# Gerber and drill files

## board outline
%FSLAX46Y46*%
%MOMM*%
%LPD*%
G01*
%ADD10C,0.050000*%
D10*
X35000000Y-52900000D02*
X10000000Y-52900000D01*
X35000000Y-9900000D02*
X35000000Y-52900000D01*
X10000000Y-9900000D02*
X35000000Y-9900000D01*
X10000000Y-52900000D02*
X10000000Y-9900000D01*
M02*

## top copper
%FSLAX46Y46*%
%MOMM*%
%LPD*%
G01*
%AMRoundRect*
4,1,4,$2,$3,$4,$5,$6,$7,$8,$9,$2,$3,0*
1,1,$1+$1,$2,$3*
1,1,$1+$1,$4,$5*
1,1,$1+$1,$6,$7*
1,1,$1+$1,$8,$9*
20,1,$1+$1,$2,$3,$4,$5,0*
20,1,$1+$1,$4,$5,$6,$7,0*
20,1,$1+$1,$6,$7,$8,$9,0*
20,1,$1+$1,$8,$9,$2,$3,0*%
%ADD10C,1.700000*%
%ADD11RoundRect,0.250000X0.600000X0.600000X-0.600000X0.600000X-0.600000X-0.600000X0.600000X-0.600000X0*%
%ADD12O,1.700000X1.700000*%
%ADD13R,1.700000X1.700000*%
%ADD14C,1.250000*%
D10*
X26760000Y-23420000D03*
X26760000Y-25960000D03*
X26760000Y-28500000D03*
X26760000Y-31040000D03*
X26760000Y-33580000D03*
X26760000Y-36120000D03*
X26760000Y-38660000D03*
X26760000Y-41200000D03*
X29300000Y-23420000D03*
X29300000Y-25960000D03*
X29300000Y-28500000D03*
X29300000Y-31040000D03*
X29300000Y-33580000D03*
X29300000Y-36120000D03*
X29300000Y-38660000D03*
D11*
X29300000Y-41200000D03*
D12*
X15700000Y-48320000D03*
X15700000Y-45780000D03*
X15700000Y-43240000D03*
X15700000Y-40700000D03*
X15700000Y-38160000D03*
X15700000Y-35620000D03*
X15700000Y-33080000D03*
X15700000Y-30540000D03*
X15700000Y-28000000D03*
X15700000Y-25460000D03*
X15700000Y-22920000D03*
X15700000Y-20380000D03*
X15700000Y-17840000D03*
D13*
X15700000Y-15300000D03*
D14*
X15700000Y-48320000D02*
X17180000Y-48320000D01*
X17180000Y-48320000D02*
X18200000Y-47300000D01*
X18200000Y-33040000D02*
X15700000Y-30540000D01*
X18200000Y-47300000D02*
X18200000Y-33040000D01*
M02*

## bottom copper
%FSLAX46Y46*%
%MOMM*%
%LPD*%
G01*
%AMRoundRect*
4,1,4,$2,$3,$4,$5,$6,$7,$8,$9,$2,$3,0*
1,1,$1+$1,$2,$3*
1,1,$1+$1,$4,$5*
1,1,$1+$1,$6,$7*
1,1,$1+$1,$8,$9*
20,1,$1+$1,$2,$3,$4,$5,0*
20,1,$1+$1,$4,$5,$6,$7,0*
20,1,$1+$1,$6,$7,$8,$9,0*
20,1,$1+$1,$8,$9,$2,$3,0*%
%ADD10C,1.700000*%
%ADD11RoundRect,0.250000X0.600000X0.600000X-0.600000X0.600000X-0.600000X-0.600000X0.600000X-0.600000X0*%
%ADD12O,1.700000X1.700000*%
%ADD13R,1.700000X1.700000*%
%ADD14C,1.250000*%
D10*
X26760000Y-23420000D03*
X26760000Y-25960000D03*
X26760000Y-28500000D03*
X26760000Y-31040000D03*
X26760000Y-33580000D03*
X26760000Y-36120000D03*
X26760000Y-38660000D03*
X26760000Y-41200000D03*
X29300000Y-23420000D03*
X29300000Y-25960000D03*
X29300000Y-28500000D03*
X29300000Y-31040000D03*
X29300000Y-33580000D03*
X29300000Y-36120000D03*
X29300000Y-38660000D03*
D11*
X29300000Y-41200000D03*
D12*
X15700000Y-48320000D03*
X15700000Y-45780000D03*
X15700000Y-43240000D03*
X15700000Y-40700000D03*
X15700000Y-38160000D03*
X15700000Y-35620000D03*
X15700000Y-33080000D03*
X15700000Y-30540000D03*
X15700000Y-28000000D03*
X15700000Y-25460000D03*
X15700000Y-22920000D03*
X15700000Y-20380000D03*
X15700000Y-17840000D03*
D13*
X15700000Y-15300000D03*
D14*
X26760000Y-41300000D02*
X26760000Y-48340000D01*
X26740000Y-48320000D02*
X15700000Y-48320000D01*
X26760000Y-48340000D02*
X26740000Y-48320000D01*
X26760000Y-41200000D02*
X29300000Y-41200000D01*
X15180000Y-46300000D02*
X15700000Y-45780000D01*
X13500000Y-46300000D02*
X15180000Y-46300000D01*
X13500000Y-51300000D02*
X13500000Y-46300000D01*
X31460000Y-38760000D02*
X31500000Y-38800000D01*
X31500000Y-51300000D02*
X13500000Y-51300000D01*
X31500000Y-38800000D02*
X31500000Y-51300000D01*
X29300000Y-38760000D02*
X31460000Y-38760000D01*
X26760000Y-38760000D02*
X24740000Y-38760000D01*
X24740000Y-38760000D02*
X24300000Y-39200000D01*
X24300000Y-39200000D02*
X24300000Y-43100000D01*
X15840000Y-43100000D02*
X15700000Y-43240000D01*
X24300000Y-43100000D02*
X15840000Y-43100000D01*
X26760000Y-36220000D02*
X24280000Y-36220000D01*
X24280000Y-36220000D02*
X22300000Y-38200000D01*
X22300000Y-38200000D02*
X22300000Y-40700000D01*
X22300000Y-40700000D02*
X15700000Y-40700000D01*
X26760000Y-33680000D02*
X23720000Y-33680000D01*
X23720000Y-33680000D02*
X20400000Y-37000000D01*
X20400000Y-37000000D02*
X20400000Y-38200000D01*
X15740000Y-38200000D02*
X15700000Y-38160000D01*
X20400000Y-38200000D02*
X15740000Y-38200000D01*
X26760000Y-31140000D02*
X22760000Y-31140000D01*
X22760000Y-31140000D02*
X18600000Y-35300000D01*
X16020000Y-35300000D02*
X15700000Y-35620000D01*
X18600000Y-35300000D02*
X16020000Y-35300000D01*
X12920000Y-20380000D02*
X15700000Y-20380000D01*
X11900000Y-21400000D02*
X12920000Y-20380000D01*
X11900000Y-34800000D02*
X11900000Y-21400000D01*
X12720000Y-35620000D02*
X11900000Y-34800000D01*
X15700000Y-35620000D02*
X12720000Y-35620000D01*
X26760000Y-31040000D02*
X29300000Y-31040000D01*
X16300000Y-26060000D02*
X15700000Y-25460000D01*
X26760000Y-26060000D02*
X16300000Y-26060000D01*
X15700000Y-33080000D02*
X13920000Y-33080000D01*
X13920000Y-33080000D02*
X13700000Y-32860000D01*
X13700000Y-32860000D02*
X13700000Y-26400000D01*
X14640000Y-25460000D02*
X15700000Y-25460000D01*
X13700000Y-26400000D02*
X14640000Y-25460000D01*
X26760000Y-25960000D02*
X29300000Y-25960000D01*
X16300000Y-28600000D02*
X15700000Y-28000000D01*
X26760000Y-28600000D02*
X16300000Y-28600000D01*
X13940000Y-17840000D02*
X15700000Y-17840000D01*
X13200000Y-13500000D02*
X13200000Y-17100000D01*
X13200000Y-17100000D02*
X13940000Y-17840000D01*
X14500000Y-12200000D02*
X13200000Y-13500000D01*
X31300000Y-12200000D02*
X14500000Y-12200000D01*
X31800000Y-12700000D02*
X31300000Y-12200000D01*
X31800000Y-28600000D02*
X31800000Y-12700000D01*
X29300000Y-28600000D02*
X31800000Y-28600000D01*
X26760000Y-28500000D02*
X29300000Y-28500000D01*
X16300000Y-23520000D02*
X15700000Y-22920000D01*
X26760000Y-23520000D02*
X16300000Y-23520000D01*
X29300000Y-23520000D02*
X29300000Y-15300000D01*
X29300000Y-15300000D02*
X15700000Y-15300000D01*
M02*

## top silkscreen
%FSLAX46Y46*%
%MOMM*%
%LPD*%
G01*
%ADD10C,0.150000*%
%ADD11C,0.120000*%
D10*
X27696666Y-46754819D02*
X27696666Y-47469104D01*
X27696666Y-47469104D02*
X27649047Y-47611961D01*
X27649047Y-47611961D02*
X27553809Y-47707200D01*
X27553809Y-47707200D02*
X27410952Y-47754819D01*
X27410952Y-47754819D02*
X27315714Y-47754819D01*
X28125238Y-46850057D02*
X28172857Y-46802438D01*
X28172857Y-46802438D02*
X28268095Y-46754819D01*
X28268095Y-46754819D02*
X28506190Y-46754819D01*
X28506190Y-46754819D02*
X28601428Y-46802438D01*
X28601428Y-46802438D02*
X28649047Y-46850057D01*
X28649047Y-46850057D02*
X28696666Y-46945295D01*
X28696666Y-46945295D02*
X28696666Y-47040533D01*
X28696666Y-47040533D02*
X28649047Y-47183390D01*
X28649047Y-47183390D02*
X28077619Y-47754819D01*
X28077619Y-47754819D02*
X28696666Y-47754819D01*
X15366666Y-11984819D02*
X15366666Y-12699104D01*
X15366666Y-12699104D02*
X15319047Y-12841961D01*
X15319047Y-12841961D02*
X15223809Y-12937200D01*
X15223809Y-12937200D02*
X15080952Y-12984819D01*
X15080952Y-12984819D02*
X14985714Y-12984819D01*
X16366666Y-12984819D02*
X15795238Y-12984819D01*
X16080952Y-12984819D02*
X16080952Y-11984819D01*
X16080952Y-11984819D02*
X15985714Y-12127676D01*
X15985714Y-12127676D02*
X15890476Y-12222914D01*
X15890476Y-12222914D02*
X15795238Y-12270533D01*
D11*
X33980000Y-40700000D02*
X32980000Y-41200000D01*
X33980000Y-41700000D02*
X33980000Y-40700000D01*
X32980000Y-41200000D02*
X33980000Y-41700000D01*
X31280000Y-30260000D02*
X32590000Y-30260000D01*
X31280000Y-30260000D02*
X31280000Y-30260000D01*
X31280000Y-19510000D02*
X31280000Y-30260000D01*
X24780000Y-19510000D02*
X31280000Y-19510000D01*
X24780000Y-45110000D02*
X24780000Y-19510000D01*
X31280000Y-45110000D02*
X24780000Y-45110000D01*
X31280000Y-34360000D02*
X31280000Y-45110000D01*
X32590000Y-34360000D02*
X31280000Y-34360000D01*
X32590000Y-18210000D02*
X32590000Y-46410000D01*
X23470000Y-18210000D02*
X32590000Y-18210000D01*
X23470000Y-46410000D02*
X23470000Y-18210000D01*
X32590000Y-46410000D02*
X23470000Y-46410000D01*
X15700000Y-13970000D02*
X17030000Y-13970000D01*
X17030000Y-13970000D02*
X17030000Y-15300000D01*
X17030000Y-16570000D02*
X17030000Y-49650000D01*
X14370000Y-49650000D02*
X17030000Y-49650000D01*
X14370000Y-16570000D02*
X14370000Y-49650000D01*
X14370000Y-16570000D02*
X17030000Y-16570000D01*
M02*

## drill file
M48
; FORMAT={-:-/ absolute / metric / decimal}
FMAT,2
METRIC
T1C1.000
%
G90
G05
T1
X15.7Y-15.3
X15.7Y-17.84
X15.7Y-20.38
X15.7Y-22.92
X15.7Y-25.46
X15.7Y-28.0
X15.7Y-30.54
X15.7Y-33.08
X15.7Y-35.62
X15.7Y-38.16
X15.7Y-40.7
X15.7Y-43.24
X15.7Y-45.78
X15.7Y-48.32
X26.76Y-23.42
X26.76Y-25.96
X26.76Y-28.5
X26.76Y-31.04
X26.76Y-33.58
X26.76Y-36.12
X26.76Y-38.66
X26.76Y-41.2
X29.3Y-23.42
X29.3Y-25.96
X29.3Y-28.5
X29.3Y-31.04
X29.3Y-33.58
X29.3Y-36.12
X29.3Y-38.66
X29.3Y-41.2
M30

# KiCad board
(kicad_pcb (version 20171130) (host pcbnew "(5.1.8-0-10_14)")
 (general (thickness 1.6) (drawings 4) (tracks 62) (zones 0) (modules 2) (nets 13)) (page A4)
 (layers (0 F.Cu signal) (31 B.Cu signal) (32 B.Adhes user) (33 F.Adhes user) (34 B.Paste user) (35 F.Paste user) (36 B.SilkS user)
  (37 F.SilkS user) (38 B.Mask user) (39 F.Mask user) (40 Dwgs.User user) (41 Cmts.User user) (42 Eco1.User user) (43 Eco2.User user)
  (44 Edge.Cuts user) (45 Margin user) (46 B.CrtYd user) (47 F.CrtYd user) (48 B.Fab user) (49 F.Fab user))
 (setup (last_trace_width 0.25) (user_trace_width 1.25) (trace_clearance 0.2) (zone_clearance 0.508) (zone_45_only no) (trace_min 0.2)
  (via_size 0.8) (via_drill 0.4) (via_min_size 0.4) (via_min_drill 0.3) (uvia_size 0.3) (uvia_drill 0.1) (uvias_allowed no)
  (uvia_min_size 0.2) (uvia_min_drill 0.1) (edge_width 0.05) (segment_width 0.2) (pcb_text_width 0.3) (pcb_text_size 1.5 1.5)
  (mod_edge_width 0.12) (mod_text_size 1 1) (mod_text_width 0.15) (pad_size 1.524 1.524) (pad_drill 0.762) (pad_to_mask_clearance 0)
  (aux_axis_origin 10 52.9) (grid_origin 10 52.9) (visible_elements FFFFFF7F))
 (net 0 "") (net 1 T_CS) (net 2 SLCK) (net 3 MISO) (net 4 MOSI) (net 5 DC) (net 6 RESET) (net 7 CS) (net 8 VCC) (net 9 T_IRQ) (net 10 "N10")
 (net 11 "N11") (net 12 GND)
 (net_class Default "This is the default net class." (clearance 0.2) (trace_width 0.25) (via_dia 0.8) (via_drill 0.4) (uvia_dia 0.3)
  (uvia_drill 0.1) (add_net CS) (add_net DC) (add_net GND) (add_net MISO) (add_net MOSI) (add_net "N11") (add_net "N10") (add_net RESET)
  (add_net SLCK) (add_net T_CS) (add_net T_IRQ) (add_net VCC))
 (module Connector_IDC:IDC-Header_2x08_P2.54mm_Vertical (layer F.Cu) (at 29.3 41.2 180)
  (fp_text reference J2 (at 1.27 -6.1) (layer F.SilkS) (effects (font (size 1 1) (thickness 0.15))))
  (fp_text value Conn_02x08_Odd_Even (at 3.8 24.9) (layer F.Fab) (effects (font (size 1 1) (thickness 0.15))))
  (fp_line (start -4.68 0.5) (end -3.68 0) (layer F.SilkS) (width 0.12))
  (fp_line (start -4.68 -0.5) (end -4.68 0.5) (layer F.SilkS) (width 0.12))
  (fp_line (start -3.68 0) (end -4.68 -0.5) (layer F.SilkS) (width 0.12))
  (fp_line (start -1.98 10.94) (end -3.29 10.94) (layer F.SilkS) (width 0.12))
  (fp_line (start -1.98 10.94) (end -1.98 10.94) (layer F.SilkS) (width 0.12))
  (fp_line (start -1.98 21.69) (end -1.98 10.94) (layer F.SilkS) (width 0.12))
  (fp_line (start 4.52 21.69) (end -1.98 21.69) (layer F.SilkS) (width 0.12))
  (fp_line (start 4.52 -3.91) (end 4.52 21.69) (layer F.SilkS) (width 0.12))
  (fp_line (start -1.98 -3.91) (end 4.52 -3.91) (layer F.SilkS) (width 0.12))
  (fp_line (start -1.98 6.84) (end -1.98 -3.91) (layer F.SilkS) (width 0.12))
  (fp_line (start -3.29 6.84) (end -1.98 6.84) (layer F.SilkS) (width 0.12))
  (fp_line (start -3.29 22.99) (end -3.29 -5.21) (layer F.SilkS) (width 0.12))
  (fp_line (start 5.83 22.99) (end -3.29 22.99) (layer F.SilkS) (width 0.12))
  (fp_line (start 5.83 -5.21) (end 5.83 22.99) (layer F.SilkS) (width 0.12))
  (fp_line (start -3.29 -5.21) (end 5.83 -5.21) (layer F.SilkS) (width 0.12))
  (pad 16 thru_hole circle (at 2.54 17.78 180) (size 1.7 1.7) (drill 1) (layers *.Cu *.Mask) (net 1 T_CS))
  (pad 14 thru_hole circle (at 2.54 15.24 180) (size 1.7 1.7) (drill 1) (layers *.Cu *.Mask) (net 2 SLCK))
  (pad 12 thru_hole circle (at 2.54 12.7 180) (size 1.7 1.7) (drill 1) (layers *.Cu *.Mask) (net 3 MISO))
  (pad 10 thru_hole circle (at 2.54 10.16 180) (size 1.7 1.7) (drill 1) (layers *.Cu *.Mask) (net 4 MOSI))
  (pad 8 thru_hole circle (at 2.54 7.62 180) (size 1.7 1.7) (drill 1) (layers *.Cu *.Mask) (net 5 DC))
  (pad 6 thru_hole circle (at 2.54 5.08 180) (size 1.7 1.7) (drill 1) (layers *.Cu *.Mask) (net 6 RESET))
  (pad 4 thru_hole circle (at 2.54 2.54 180) (size 1.7 1.7) (drill 1) (layers *.Cu *.Mask) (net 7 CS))
  (pad 2 thru_hole circle (at 2.54 0 180) (size 1.7 1.7) (drill 1) (layers *.Cu *.Mask) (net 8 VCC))
  (pad 15 thru_hole circle (at 0 17.78 180) (size 1.7 1.7) (drill 1) (layers *.Cu *.Mask) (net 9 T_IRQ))
  (pad 13 thru_hole circle (at 0 15.24 180) (size 1.7 1.7) (drill 1) (layers *.Cu *.Mask) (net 2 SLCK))
  (pad 11 thru_hole circle (at 0 12.7 180) (size 1.7 1.7) (drill 1) (layers *.Cu *.Mask) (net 3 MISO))
  (pad 9 thru_hole circle (at 0 10.16 180) (size 1.7 1.7) (drill 1) (layers *.Cu *.Mask) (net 4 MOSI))
  (pad 7 thru_hole circle (at 0 7.62 180) (size 1.7 1.7) (drill 1) (layers *.Cu *.Mask) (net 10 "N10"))
  (pad 5 thru_hole circle (at 0 5.08 180) (size 1.7 1.7) (drill 1) (layers *.Cu *.Mask) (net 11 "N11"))
  (pad 3 thru_hole circle (at 0 2.54 180) (size 1.7 1.7) (drill 1) (layers *.Cu *.Mask) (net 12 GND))
  (pad 1 thru_hole roundrect (at 0 0 180) (size 1.7 1.7) (drill 1) (layers *.Cu *.Mask) (roundrect_rratio 0.1470588235294118) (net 8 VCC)))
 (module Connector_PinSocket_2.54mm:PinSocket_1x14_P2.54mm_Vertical (layer F.Cu) (at 15.7 15.3)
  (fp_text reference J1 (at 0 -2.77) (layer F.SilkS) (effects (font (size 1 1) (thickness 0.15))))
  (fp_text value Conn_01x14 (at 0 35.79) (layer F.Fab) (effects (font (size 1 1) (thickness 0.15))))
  (fp_line (start 0 -1.33) (end 1.33 -1.33) (layer F.SilkS) (width 0.12))
  (fp_line (start 1.33 -1.33) (end 1.33 0) (layer F.SilkS) (width 0.12))
  (fp_line (start 1.33 1.27) (end 1.33 34.35) (layer F.SilkS) (width 0.12))
  (fp_line (start -1.33 34.35) (end 1.33 34.35) (layer F.SilkS) (width 0.12))
  (fp_line (start -1.33 1.27) (end -1.33 34.35) (layer F.SilkS) (width 0.12))
  (fp_line (start -1.33 1.27) (end 1.33 1.27) (layer F.SilkS) (width 0.12))
  (pad 14 thru_hole oval (at 0 33.02) (size 1.7 1.7) (drill 1) (layers *.Cu *.Mask) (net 8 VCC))
  (pad 13 thru_hole oval (at 0 30.48) (size 1.7 1.7) (drill 1) (layers *.Cu *.Mask) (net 12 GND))
  (pad 12 thru_hole oval (at 0 27.94) (size 1.7 1.7) (drill 1) (layers *.Cu *.Mask) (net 7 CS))
  (pad 11 thru_hole oval (at 0 25.4) (size 1.7 1.7) (drill 1) (layers *.Cu *.Mask) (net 6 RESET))
  (pad 10 thru_hole oval (at 0 22.86) (size 1.7 1.7) (drill 1) (layers *.Cu *.Mask) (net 5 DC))
  (pad 9 thru_hole oval (at 0 20.32) (size 1.7 1.7) (drill 1) (layers *.Cu *.Mask) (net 4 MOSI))
  (pad 8 thru_hole oval (at 0 17.78) (size 1.7 1.7) (drill 1) (layers *.Cu *.Mask) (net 2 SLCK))
  (pad 7 thru_hole oval (at 0 15.24) (size 1.7 1.7) (drill 1) (layers *.Cu *.Mask) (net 8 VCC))
  (pad 6 thru_hole oval (at 0 12.7) (size 1.7 1.7) (drill 1) (layers *.Cu *.Mask) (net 3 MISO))
  (pad 5 thru_hole oval (at 0 10.16) (size 1.7 1.7) (drill 1) (layers *.Cu *.Mask) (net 2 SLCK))
  (pad 4 thru_hole oval (at 0 7.62) (size 1.7 1.7) (drill 1) (layers *.Cu *.Mask) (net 1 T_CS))
  (pad 3 thru_hole oval (at 0 5.08) (size 1.7 1.7) (drill 1) (layers *.Cu *.Mask) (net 4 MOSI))
  (pad 2 thru_hole oval (at 0 2.54) (size 1.7 1.7) (drill 1) (layers *.Cu *.Mask) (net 3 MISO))
  (pad 1 thru_hole rect (at 0 0) (size 1.7 1.7) (drill 1) (layers *.Cu *.Mask) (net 9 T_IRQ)))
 (gr_line (start 35 52.9) (end 10 52.9) (layer Edge.Cuts) (width 0.05))
 (gr_line (start 35 9.9) (end 35 52.9) (layer Edge.Cuts) (width 0.05))
 (gr_line (start 10 9.9) (end 35 9.9) (layer Edge.Cuts) (width 0.05))
 (gr_line (start 10 52.9) (end 10 9.9) (layer Edge.Cuts) (width 0.05))
 (segment (start 26.76 41.3) (end 26.76 48.34) (width 1.25) (layer B.Cu) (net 8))
 (segment (start 26.74 48.32) (end 15.7 48.32) (width 1.25) (layer B.Cu) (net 8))
 (segment (start 26.76 48.34) (end 26.74 48.32) (width 1.25) (layer B.Cu) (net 8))
 (segment (start 26.76 41.2) (end 29.3 41.2) (width 1.25) (layer B.Cu) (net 8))
 (segment (start 15.7 48.32) (end 17.18 48.32) (width 1.25) (layer F.Cu) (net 8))
 (segment (start 17.18 48.32) (end 18.2 47.3) (width 1.25) (layer F.Cu) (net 8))
 (segment (start 18.2 33.04) (end 15.7 30.54) (width 1.25) (layer F.Cu) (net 8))
 (segment (start 18.2 47.3) (end 18.2 33.04) (width 1.25) (layer F.Cu) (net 8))
 (segment (start 15.18 46.3) (end 15.7 45.78) (width 1.25) (layer B.Cu) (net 12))
 (segment (start 13.5 46.3) (end 15.18 46.3) (width 1.25) (layer B.Cu) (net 12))
 (segment (start 13.5 51.3) (end 13.5 46.3) (width 1.25) (layer B.Cu) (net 12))
 (segment (start 31.46 38.76) (end 31.5 38.8) (width 1.25) (layer B.Cu) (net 12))
 (segment (start 31.5 51.3) (end 13.5 51.3) (width 1.25) (layer B.Cu) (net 12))
 (segment (start 31.5 38.8) (end 31.5 51.3) (width 1.25) (layer B.Cu) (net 12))
 (segment (start 29.3 38.76) (end 31.46 38.76) (width 1.25) (layer B.Cu) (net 12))
 (segment (start 26.76 38.76) (end 24.74 38.76) (width 1.25) (layer B.Cu) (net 7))
 (segment (start 24.74 38.76) (end 24.3 39.2) (width 1.25) (layer B.Cu) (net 7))
 (segment (start 24.3 39.2) (end 24.3 43.1) (width 1.25) (layer B.Cu) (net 7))
 (segment (start 15.84 43.1) (end 15.7 43.24) (width 1.25) (layer B.Cu) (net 7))
 (segment (start 24.3 43.1) (end 15.84 43.1) (width 1.25) (layer B.Cu) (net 7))
 (segment (start 26.76 36.22) (end 24.28 36.22) (width 1.25) (layer B.Cu) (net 6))
 (segment (start 24.28 36.22) (end 22.3 38.2) (width 1.25) (layer B.Cu) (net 6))
 (segment (start 22.3 38.2) (end 22.3 40.7) (width 1.25) (layer B.Cu) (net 6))
 (segment (start 22.3 40.7) (end 15.7 40.7) (width 1.25) (layer B.Cu) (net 6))
 (segment (start 26.76 33.68) (end 23.72 33.68) (width 1.25) (layer B.Cu) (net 5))
 (segment (start 23.72 33.68) (end 20.4 37) (width 1.25) (layer B.Cu) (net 5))
 (segment (start 20.4 37) (end 20.4 38.2) (width 1.25) (layer B.Cu) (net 5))
 (segment (start 15.74 38.2) (end 15.7 38.16) (width 1.25) (layer B.Cu) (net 5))
 (segment (start 20.4 38.2) (end 15.74 38.2) (width 1.25) (layer B.Cu) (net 5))
 (segment (start 26.76 31.14) (end 22.76 31.14) (width 1.25) (layer B.Cu) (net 4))
 (segment (start 22.76 31.14) (end 18.6 35.3) (width 1.25) (layer B.Cu) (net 4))
 (segment (start 16.02 35.3) (end 15.7 35.62) (width 1.25) (layer B.Cu) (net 4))
 (segment (start 18.6 35.3) (end 16.02 35.3) (width 1.25) (layer B.Cu) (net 4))
 (segment (start 12.92 20.38) (end 15.7 20.38) (width 1.25) (layer B.Cu) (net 4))
 (segment (start 11.9 21.4) (end 12.92 20.38) (width 1.25) (layer B.Cu) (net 4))
 (segment (start 11.9 34.8) (end 11.9 21.4) (width 1.25) (layer B.Cu) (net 4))
 (segment (start 12.72 35.62) (end 11.9 34.8) (width 1.25) (layer B.Cu) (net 4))
 (segment (start 15.7 35.62) (end 12.72 35.62) (width 1.25) (layer B.Cu) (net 4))
 (segment (start 26.76 31.04) (end 29.3 31.04) (width 1.25) (layer B.Cu) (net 4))
 (segment (start 16.3 26.06) (end 15.7 25.46) (width 1.25) (layer B.Cu) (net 2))
 (segment (start 26.76 26.06) (end 16.3 26.06) (width 1.25) (layer B.Cu) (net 2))
 (segment (start 15.7 33.08) (end 13.92 33.08) (width 1.25) (layer B.Cu) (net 2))
 (segment (start 13.92 33.08) (end 13.7 32.86) (width 1.25) (layer B.Cu) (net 2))
 (segment (start 13.7 32.86) (end 13.7 26.4) (width 1.25) (layer B.Cu) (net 2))
 (segment (start 14.64 25.46) (end 15.7 25.46) (width 1.25) (layer B.Cu) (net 2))
 (segment (start 13.7 26.4) (end 14.64 25.46) (width 1.25) (layer B.Cu) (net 2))
 (segment (start 26.76 25.96) (end 29.3 25.96) (width 1.25) (layer B.Cu) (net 2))
 (segment (start 16.3 28.6) (end 15.7 28) (width 1.25) (layer B.Cu) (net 3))
 (segment (start 26.76 28.6) (end 16.3 28.6) (width 1.25) (layer B.Cu) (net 3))
 (segment (start 13.94 17.84) (end 15.7 17.84) (width 1.25) (layer B.Cu) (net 3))
 (segment (start 13.2 13.5) (end 13.2 17.1) (width 1.25) (layer B.Cu) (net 3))
 (segment (start 13.2 17.1) (end 13.94 17.84) (width 1.25) (layer B.Cu) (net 3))
 (segment (start 14.5 12.2) (end 13.2 13.5) (width 1.25) (layer B.Cu) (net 3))
 (segment (start 31.3 12.2) (end 14.5 12.2) (width 1.25) (layer B.Cu) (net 3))
 (segment (start 31.8 12.7) (end 31.3 12.2) (width 1.25) (layer B.Cu) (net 3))
 (segment (start 31.8 28.6) (end 31.8 12.7) (width 1.25) (layer B.Cu) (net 3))
 (segment (start 29.3 28.6) (end 31.8 28.6) (width 1.25) (layer B.Cu) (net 3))
 (segment (start 26.76 28.5) (end 29.3 28.5) (width 1.25) (layer B.Cu) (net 3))
 (segment (start 16.3 23.52) (end 15.7 22.92) (width 1.25) (layer B.Cu) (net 1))
 (segment (start 26.76 23.52) (end 16.3 23.52) (width 1.25) (layer B.Cu) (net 1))
 (segment (start 29.3 23.52) (end 29.3 15.3) (width 1.25) (layer B.Cu) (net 9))
 (segment (start 29.3 15.3) (end 15.7 15.3) (width 1.25) (layer B.Cu) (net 9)))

